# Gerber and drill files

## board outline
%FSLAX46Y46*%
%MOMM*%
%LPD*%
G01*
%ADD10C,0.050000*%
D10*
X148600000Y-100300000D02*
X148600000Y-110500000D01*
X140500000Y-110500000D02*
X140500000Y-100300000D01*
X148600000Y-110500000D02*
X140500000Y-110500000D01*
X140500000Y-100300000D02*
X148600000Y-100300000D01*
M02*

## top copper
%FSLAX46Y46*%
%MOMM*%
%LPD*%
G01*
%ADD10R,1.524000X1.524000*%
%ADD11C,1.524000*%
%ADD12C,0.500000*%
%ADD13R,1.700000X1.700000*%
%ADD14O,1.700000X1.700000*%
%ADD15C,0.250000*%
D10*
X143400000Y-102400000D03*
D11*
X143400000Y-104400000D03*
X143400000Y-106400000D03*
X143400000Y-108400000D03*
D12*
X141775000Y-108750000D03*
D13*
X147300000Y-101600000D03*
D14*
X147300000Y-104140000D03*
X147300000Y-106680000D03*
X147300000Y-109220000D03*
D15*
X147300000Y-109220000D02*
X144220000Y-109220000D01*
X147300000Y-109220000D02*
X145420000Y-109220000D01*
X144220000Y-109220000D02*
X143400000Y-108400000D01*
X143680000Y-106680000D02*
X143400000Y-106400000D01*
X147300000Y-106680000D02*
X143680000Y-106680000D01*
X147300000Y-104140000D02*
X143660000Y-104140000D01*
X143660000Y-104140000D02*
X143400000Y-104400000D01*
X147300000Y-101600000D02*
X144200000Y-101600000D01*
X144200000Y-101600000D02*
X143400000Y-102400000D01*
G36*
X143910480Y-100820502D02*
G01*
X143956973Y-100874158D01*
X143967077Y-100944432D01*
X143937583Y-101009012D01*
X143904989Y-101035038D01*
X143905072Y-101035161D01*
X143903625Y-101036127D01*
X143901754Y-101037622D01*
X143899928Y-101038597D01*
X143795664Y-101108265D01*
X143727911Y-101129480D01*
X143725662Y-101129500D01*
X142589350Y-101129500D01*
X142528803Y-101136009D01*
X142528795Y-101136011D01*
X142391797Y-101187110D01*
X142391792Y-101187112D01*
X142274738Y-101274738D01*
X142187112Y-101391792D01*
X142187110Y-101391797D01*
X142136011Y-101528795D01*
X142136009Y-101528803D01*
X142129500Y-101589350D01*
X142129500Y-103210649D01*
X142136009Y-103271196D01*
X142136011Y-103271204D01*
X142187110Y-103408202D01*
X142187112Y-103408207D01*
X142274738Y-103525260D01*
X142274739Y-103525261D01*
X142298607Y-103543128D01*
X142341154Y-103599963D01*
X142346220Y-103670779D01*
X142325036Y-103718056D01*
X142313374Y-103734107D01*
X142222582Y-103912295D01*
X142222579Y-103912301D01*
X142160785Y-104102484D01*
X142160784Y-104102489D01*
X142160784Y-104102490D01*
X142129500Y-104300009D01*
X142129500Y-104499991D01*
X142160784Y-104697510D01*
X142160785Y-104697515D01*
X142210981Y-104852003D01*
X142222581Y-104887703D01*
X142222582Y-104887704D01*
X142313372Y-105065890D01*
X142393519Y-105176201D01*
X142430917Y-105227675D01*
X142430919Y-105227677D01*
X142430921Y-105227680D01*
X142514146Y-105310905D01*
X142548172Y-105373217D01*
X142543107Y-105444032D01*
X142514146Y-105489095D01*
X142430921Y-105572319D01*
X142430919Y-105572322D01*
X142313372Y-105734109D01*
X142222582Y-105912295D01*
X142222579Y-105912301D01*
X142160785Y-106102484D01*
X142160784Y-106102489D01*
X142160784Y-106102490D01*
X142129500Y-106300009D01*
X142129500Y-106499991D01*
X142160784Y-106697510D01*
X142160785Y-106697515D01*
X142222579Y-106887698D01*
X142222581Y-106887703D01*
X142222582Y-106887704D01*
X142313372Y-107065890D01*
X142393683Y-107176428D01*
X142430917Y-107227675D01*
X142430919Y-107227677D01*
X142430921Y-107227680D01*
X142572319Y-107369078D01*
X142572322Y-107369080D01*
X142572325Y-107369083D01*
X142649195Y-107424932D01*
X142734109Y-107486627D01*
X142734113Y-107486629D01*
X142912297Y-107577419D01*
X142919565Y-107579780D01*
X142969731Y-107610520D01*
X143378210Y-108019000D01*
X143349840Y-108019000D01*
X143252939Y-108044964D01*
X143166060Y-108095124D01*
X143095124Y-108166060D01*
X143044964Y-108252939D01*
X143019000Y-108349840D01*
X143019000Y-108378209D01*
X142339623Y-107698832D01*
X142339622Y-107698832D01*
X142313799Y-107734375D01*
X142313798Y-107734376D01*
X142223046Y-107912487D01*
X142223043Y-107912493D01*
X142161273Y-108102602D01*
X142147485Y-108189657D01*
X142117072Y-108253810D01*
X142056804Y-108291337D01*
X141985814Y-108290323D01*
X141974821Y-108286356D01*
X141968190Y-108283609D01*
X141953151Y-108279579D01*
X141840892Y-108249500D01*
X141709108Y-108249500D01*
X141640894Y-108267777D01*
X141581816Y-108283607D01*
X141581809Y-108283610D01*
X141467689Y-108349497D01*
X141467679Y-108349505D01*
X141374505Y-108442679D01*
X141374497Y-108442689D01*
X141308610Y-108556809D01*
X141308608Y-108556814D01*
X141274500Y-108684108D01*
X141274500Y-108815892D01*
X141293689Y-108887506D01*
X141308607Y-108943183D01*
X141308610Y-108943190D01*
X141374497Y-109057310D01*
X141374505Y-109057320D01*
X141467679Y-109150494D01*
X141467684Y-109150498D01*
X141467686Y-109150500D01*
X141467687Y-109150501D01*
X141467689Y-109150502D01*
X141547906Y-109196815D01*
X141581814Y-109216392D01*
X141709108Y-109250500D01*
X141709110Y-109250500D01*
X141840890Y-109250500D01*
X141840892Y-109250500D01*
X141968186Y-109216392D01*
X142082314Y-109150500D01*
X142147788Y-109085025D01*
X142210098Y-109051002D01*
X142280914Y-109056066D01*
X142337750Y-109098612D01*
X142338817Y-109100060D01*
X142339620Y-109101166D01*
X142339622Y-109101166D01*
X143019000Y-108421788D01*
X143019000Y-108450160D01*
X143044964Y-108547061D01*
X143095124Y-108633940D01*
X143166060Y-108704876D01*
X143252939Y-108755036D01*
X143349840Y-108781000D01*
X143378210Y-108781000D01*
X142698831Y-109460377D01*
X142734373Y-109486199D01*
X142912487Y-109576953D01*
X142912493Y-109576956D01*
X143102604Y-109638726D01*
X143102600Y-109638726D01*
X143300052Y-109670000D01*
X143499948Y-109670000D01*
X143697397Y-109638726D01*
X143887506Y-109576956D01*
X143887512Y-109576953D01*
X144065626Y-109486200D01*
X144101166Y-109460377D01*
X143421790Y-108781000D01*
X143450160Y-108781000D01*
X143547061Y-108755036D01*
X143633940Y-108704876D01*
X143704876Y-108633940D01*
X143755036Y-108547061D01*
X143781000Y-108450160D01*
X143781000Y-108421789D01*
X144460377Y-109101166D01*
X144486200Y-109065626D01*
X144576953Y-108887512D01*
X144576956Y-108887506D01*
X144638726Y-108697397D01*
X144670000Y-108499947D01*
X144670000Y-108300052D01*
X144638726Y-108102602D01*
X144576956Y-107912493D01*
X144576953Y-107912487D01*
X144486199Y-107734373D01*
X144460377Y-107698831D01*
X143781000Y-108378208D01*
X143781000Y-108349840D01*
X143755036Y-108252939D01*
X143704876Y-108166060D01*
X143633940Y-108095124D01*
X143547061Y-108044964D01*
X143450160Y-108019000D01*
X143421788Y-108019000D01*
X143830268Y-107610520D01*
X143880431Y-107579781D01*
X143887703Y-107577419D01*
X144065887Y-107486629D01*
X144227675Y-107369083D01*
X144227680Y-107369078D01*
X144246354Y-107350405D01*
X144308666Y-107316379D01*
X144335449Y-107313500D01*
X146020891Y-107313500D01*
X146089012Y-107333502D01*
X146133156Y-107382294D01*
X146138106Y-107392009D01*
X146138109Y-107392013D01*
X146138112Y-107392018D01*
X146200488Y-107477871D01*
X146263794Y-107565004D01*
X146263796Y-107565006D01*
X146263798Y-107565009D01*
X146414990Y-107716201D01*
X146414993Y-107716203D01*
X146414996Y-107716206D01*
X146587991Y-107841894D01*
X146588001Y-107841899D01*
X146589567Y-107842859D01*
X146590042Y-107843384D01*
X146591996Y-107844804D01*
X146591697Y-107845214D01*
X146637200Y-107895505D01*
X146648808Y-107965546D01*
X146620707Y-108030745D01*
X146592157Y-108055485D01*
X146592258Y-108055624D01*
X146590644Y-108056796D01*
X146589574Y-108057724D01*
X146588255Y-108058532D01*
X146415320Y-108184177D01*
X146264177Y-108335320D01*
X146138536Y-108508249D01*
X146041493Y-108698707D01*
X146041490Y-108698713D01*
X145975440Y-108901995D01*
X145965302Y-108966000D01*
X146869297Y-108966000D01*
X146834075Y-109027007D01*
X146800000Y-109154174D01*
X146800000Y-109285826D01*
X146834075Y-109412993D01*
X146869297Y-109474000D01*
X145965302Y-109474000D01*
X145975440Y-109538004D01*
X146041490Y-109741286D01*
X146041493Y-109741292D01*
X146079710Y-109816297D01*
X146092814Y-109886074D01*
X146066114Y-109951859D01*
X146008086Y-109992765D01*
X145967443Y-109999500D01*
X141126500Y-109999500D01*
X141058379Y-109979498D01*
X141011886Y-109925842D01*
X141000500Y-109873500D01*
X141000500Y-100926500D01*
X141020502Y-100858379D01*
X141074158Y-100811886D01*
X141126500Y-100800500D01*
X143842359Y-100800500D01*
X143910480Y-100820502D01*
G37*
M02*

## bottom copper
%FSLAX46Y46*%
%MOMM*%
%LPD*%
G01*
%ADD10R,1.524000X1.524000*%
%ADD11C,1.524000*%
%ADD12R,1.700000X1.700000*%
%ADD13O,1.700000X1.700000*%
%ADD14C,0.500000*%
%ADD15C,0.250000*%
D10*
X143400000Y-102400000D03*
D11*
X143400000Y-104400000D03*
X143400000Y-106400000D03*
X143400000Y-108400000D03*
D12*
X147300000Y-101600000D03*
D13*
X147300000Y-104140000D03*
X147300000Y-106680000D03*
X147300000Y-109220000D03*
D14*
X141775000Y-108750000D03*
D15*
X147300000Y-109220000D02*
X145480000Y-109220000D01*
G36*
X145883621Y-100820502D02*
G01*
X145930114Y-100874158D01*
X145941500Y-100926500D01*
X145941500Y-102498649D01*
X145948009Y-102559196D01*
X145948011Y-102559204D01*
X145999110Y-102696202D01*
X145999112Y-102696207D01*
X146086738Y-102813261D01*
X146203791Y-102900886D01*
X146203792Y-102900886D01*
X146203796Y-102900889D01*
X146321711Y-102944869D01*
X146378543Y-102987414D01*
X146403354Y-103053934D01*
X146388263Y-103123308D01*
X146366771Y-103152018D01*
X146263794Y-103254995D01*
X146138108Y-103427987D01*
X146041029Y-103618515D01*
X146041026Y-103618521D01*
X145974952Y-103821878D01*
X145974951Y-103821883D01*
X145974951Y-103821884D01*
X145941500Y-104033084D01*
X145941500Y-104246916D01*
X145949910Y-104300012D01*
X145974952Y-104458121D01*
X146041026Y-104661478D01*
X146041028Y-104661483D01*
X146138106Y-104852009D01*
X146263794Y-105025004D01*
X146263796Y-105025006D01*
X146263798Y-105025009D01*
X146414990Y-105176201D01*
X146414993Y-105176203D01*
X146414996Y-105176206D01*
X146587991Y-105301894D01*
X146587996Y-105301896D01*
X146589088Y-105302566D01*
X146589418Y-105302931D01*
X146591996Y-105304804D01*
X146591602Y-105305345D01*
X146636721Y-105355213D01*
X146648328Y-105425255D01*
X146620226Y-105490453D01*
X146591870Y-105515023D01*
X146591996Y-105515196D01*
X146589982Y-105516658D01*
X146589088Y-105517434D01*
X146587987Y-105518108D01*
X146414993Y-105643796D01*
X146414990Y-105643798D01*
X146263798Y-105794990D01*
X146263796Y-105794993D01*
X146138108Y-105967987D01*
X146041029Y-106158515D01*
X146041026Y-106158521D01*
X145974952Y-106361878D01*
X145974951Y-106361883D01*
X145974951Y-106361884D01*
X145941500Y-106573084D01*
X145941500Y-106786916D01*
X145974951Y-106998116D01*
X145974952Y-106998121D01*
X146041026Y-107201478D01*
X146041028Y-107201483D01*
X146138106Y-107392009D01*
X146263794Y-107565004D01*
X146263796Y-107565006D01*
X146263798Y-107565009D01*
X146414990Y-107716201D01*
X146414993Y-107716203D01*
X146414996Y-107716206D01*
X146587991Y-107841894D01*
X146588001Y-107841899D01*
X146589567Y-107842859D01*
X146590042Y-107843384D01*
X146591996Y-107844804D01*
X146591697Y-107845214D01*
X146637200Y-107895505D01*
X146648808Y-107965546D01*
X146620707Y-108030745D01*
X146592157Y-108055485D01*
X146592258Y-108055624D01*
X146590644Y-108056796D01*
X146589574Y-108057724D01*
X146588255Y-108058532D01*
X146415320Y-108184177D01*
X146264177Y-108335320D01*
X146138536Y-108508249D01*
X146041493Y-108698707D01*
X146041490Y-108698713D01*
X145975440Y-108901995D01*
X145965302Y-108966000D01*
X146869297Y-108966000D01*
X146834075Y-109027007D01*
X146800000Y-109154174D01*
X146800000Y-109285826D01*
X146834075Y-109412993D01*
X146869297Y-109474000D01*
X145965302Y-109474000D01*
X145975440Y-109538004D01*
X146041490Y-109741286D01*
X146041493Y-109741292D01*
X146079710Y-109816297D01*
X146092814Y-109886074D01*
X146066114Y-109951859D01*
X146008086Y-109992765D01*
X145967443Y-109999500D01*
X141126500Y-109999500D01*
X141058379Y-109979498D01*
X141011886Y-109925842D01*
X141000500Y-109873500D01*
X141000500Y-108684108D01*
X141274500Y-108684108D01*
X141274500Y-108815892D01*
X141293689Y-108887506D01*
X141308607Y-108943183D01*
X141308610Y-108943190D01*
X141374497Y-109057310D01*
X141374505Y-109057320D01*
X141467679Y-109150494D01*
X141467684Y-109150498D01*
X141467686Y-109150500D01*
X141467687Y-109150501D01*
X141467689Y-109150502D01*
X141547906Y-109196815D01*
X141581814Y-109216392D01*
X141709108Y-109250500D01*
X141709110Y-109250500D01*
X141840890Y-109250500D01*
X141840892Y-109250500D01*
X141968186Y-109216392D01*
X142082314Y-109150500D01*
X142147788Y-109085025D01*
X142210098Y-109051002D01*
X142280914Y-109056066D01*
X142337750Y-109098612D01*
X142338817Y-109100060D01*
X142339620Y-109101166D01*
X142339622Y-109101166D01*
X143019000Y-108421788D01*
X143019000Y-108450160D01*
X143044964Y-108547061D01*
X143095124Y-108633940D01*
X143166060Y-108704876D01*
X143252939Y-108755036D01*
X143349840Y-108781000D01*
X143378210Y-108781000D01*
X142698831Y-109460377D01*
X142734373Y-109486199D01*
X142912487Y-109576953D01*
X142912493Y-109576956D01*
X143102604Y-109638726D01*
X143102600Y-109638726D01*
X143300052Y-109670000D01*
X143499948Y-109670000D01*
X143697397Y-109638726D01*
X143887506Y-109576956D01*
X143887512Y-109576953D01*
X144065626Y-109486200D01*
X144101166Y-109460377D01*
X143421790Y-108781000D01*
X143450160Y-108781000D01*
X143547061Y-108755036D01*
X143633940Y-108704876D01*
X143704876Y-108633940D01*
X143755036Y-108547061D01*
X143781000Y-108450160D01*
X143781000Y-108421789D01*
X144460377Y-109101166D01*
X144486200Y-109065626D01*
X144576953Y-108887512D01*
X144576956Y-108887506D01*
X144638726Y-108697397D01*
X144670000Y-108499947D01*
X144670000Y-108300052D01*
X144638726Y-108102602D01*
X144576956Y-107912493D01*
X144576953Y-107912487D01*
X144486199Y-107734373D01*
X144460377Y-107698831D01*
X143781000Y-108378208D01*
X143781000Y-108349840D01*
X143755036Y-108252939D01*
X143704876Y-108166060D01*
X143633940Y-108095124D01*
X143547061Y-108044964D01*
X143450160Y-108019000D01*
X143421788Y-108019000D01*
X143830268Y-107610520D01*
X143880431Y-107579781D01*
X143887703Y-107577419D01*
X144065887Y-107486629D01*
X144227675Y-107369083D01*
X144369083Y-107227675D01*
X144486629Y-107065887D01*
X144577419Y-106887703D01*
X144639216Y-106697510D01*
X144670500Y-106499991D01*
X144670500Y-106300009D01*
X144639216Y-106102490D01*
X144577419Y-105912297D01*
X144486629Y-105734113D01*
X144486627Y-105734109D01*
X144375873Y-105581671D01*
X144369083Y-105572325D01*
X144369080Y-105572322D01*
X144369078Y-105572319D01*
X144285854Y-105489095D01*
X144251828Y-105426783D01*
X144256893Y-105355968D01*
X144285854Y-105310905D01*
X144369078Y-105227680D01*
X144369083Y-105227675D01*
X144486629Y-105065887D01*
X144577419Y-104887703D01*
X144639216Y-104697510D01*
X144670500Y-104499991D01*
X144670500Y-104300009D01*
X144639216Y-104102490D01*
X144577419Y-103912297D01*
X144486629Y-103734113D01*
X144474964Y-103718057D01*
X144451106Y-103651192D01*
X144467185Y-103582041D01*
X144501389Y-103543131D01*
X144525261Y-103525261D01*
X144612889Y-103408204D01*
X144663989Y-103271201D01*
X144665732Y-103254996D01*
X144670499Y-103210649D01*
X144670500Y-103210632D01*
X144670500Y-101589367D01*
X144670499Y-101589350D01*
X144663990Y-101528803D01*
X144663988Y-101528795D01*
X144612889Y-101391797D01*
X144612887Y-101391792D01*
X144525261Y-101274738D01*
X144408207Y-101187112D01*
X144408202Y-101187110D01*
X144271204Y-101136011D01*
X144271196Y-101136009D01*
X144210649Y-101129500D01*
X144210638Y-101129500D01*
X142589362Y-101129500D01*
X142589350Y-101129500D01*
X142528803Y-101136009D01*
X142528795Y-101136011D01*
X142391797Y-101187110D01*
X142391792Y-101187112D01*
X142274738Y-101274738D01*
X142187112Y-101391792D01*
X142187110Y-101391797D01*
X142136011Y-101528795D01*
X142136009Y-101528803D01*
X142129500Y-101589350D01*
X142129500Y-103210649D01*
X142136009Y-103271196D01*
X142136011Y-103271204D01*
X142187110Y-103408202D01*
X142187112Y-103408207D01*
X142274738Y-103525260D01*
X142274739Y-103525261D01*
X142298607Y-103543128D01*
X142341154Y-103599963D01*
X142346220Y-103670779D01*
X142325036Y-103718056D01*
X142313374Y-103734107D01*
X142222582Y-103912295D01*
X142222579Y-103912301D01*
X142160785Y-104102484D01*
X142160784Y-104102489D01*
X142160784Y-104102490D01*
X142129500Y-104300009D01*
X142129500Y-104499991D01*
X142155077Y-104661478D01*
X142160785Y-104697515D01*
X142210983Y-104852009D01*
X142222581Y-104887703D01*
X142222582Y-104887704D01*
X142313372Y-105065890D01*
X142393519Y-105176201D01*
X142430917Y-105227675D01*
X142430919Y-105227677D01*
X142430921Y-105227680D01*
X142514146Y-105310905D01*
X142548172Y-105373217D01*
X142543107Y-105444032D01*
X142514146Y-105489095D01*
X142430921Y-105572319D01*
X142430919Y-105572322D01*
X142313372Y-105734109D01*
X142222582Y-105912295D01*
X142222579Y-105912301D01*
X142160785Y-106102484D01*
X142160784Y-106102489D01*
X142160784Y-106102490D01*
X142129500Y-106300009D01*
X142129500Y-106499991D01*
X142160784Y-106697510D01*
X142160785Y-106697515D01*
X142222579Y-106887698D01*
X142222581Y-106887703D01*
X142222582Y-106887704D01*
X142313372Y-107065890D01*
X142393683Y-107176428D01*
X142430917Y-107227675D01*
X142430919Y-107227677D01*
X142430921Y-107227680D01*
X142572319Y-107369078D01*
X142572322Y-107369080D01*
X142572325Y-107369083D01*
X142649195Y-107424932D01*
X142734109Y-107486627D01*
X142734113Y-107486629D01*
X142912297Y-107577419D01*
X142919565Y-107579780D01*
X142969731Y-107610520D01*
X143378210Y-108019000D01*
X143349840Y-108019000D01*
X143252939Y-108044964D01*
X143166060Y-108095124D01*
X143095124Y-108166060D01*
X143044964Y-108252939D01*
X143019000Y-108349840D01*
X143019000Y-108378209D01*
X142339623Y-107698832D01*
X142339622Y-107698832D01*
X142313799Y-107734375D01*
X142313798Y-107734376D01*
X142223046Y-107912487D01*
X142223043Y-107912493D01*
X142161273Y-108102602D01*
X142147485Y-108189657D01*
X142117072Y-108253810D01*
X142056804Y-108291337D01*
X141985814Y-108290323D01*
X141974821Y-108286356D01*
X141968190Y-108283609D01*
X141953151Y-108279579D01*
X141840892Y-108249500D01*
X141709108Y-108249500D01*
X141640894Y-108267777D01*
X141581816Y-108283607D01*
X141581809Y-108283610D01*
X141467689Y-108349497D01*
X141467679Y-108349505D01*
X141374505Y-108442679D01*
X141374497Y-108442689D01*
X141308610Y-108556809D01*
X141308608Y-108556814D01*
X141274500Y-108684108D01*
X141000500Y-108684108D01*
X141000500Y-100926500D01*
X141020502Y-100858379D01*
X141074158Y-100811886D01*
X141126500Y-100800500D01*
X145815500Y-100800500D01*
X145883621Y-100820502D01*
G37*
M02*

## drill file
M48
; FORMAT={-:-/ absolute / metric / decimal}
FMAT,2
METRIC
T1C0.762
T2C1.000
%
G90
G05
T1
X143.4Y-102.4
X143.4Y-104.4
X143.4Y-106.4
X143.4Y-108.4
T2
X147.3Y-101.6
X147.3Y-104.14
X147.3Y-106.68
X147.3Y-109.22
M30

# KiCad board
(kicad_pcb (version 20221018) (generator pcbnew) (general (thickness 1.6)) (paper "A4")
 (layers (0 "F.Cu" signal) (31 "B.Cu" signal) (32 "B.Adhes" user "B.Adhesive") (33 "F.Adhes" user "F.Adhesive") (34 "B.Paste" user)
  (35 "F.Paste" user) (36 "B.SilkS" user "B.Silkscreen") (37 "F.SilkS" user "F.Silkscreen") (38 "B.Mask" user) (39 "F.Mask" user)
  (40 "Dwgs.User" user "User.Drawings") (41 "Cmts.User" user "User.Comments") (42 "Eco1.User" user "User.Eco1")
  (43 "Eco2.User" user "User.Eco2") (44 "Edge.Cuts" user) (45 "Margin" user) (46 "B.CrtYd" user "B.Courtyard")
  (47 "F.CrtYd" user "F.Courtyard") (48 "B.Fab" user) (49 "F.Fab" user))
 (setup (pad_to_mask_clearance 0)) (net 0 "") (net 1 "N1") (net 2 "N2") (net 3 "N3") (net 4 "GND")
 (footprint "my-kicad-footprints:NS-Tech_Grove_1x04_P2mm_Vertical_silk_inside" (layer "F.Cu") (at 143.4 102.4)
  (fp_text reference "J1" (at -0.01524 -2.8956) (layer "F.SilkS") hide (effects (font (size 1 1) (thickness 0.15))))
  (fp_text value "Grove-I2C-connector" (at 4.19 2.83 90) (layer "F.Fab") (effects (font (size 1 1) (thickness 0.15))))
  (pad "1" thru_hole rect (at 0 0) (size 1.524 1.524) (drill 0.762) (layers "*.Cu" "*.Mask") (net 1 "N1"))
  (pad "2" thru_hole circle (at 0 2) (size 1.524 1.524) (drill 0.762) (layers "*.Cu" "*.Mask") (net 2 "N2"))
  (pad "3" thru_hole circle (at 0 4) (size 1.524 1.524) (drill 0.762) (layers "*.Cu" "*.Mask") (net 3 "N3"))
  (pad "4" thru_hole circle (at 0 6) (size 1.524 1.524) (drill 0.762) (layers "*.Cu" "*.Mask") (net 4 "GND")))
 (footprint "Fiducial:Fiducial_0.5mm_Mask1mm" (layer "F.Cu") (at 141.775 108.75)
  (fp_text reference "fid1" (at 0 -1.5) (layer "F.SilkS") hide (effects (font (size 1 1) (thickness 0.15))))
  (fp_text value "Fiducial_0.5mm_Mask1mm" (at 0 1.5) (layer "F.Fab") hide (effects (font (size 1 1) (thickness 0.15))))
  (pad "" smd circle (at 0 0) (size 0.5 0.5) (layers "F.Cu" "F.Mask") (solder_mask_margin 0.25) (clearance 0.25)))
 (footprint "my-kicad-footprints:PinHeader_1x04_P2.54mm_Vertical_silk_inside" (layer "B.Cu") (at 147.3 101.6 180)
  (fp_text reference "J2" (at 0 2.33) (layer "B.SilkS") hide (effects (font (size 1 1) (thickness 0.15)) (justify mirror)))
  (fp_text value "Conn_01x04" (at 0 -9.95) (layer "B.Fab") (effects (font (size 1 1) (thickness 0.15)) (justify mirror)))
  (pad "1" thru_hole rect (at 0 0 180) (size 1.7 1.7) (drill 1) (layers "*.Cu" "*.Mask") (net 1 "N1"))
  (pad "2" thru_hole oval (at 0 -2.54 180) (size 1.7 1.7) (drill 1) (layers "*.Cu" "*.Mask") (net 2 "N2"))
  (pad "3" thru_hole oval (at 0 -5.08 180) (size 1.7 1.7) (drill 1) (layers "*.Cu" "*.Mask") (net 3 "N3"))
  (pad "4" thru_hole oval (at 0 -7.62 180) (size 1.7 1.7) (drill 1) (layers "*.Cu" "*.Mask") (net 4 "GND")))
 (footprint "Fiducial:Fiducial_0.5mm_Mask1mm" (layer "B.Cu") (at 141.775 108.75)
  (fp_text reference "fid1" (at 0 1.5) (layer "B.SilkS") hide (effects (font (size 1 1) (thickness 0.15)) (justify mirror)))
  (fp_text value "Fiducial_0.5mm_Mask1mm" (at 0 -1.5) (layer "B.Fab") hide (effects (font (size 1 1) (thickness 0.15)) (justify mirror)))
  (pad "" smd circle (at 0 0) (size 0.5 0.5) (layers "B.Cu" "B.Mask") (solder_mask_margin 0.25) (clearance 0.25)))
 (gr_line (start 148.6 100.3) (end 148.6 110.5) (stroke (width 0.05) (type solid)) (layer "Edge.Cuts"))
 (gr_line (start 140.5 110.5) (end 140.5 100.3) (stroke (width 0.05) (type solid)) (layer "Edge.Cuts"))
 (gr_line (start 148.6 110.5) (end 140.5 110.5) (stroke (width 0.05) (type solid)) (layer "Edge.Cuts"))
 (gr_line (start 140.5 100.3) (end 148.6 100.3) (stroke (width 0.05) (type solid)) (layer "Edge.Cuts"))
 (segment (start 147.3 109.22) (end 144.22 109.22) (width 0.25) (layer "F.Cu") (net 4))
 (segment (start 147.3 109.22) (end 145.42 109.22) (width 0.25) (layer "F.Cu") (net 4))
 (segment (start 144.22 109.22) (end 143.4 108.4) (width 0.25) (layer "F.Cu") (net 4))
 (segment (start 147.3 109.22) (end 145.48 109.22) (width 0.25) (layer "B.Cu") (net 4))
 (segment (start 143.68 106.68) (end 143.4 106.4) (width 0.25) (layer "F.Cu") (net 3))
 (segment (start 147.3 106.68) (end 143.68 106.68) (width 0.25) (layer "F.Cu") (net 3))
 (segment (start 147.3 104.14) (end 143.66 104.14) (width 0.25) (layer "F.Cu") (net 2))
 (segment (start 143.66 104.14) (end 143.4 104.4) (width 0.25) (layer "F.Cu") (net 2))
 (segment (start 147.3 101.6) (end 144.2 101.6) (width 0.25) (layer "F.Cu") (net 1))
 (segment (start 144.2 101.6) (end 143.4 102.4) (width 0.25) (layer "F.Cu") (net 1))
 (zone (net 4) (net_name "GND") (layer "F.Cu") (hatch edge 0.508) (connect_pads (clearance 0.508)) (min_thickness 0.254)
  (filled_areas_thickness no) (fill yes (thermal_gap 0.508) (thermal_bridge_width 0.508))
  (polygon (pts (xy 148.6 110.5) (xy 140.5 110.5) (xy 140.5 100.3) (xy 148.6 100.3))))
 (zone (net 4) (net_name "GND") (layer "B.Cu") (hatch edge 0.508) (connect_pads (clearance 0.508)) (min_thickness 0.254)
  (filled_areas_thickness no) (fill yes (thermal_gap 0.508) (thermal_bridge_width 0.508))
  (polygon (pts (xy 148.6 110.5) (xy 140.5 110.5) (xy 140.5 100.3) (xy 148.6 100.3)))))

